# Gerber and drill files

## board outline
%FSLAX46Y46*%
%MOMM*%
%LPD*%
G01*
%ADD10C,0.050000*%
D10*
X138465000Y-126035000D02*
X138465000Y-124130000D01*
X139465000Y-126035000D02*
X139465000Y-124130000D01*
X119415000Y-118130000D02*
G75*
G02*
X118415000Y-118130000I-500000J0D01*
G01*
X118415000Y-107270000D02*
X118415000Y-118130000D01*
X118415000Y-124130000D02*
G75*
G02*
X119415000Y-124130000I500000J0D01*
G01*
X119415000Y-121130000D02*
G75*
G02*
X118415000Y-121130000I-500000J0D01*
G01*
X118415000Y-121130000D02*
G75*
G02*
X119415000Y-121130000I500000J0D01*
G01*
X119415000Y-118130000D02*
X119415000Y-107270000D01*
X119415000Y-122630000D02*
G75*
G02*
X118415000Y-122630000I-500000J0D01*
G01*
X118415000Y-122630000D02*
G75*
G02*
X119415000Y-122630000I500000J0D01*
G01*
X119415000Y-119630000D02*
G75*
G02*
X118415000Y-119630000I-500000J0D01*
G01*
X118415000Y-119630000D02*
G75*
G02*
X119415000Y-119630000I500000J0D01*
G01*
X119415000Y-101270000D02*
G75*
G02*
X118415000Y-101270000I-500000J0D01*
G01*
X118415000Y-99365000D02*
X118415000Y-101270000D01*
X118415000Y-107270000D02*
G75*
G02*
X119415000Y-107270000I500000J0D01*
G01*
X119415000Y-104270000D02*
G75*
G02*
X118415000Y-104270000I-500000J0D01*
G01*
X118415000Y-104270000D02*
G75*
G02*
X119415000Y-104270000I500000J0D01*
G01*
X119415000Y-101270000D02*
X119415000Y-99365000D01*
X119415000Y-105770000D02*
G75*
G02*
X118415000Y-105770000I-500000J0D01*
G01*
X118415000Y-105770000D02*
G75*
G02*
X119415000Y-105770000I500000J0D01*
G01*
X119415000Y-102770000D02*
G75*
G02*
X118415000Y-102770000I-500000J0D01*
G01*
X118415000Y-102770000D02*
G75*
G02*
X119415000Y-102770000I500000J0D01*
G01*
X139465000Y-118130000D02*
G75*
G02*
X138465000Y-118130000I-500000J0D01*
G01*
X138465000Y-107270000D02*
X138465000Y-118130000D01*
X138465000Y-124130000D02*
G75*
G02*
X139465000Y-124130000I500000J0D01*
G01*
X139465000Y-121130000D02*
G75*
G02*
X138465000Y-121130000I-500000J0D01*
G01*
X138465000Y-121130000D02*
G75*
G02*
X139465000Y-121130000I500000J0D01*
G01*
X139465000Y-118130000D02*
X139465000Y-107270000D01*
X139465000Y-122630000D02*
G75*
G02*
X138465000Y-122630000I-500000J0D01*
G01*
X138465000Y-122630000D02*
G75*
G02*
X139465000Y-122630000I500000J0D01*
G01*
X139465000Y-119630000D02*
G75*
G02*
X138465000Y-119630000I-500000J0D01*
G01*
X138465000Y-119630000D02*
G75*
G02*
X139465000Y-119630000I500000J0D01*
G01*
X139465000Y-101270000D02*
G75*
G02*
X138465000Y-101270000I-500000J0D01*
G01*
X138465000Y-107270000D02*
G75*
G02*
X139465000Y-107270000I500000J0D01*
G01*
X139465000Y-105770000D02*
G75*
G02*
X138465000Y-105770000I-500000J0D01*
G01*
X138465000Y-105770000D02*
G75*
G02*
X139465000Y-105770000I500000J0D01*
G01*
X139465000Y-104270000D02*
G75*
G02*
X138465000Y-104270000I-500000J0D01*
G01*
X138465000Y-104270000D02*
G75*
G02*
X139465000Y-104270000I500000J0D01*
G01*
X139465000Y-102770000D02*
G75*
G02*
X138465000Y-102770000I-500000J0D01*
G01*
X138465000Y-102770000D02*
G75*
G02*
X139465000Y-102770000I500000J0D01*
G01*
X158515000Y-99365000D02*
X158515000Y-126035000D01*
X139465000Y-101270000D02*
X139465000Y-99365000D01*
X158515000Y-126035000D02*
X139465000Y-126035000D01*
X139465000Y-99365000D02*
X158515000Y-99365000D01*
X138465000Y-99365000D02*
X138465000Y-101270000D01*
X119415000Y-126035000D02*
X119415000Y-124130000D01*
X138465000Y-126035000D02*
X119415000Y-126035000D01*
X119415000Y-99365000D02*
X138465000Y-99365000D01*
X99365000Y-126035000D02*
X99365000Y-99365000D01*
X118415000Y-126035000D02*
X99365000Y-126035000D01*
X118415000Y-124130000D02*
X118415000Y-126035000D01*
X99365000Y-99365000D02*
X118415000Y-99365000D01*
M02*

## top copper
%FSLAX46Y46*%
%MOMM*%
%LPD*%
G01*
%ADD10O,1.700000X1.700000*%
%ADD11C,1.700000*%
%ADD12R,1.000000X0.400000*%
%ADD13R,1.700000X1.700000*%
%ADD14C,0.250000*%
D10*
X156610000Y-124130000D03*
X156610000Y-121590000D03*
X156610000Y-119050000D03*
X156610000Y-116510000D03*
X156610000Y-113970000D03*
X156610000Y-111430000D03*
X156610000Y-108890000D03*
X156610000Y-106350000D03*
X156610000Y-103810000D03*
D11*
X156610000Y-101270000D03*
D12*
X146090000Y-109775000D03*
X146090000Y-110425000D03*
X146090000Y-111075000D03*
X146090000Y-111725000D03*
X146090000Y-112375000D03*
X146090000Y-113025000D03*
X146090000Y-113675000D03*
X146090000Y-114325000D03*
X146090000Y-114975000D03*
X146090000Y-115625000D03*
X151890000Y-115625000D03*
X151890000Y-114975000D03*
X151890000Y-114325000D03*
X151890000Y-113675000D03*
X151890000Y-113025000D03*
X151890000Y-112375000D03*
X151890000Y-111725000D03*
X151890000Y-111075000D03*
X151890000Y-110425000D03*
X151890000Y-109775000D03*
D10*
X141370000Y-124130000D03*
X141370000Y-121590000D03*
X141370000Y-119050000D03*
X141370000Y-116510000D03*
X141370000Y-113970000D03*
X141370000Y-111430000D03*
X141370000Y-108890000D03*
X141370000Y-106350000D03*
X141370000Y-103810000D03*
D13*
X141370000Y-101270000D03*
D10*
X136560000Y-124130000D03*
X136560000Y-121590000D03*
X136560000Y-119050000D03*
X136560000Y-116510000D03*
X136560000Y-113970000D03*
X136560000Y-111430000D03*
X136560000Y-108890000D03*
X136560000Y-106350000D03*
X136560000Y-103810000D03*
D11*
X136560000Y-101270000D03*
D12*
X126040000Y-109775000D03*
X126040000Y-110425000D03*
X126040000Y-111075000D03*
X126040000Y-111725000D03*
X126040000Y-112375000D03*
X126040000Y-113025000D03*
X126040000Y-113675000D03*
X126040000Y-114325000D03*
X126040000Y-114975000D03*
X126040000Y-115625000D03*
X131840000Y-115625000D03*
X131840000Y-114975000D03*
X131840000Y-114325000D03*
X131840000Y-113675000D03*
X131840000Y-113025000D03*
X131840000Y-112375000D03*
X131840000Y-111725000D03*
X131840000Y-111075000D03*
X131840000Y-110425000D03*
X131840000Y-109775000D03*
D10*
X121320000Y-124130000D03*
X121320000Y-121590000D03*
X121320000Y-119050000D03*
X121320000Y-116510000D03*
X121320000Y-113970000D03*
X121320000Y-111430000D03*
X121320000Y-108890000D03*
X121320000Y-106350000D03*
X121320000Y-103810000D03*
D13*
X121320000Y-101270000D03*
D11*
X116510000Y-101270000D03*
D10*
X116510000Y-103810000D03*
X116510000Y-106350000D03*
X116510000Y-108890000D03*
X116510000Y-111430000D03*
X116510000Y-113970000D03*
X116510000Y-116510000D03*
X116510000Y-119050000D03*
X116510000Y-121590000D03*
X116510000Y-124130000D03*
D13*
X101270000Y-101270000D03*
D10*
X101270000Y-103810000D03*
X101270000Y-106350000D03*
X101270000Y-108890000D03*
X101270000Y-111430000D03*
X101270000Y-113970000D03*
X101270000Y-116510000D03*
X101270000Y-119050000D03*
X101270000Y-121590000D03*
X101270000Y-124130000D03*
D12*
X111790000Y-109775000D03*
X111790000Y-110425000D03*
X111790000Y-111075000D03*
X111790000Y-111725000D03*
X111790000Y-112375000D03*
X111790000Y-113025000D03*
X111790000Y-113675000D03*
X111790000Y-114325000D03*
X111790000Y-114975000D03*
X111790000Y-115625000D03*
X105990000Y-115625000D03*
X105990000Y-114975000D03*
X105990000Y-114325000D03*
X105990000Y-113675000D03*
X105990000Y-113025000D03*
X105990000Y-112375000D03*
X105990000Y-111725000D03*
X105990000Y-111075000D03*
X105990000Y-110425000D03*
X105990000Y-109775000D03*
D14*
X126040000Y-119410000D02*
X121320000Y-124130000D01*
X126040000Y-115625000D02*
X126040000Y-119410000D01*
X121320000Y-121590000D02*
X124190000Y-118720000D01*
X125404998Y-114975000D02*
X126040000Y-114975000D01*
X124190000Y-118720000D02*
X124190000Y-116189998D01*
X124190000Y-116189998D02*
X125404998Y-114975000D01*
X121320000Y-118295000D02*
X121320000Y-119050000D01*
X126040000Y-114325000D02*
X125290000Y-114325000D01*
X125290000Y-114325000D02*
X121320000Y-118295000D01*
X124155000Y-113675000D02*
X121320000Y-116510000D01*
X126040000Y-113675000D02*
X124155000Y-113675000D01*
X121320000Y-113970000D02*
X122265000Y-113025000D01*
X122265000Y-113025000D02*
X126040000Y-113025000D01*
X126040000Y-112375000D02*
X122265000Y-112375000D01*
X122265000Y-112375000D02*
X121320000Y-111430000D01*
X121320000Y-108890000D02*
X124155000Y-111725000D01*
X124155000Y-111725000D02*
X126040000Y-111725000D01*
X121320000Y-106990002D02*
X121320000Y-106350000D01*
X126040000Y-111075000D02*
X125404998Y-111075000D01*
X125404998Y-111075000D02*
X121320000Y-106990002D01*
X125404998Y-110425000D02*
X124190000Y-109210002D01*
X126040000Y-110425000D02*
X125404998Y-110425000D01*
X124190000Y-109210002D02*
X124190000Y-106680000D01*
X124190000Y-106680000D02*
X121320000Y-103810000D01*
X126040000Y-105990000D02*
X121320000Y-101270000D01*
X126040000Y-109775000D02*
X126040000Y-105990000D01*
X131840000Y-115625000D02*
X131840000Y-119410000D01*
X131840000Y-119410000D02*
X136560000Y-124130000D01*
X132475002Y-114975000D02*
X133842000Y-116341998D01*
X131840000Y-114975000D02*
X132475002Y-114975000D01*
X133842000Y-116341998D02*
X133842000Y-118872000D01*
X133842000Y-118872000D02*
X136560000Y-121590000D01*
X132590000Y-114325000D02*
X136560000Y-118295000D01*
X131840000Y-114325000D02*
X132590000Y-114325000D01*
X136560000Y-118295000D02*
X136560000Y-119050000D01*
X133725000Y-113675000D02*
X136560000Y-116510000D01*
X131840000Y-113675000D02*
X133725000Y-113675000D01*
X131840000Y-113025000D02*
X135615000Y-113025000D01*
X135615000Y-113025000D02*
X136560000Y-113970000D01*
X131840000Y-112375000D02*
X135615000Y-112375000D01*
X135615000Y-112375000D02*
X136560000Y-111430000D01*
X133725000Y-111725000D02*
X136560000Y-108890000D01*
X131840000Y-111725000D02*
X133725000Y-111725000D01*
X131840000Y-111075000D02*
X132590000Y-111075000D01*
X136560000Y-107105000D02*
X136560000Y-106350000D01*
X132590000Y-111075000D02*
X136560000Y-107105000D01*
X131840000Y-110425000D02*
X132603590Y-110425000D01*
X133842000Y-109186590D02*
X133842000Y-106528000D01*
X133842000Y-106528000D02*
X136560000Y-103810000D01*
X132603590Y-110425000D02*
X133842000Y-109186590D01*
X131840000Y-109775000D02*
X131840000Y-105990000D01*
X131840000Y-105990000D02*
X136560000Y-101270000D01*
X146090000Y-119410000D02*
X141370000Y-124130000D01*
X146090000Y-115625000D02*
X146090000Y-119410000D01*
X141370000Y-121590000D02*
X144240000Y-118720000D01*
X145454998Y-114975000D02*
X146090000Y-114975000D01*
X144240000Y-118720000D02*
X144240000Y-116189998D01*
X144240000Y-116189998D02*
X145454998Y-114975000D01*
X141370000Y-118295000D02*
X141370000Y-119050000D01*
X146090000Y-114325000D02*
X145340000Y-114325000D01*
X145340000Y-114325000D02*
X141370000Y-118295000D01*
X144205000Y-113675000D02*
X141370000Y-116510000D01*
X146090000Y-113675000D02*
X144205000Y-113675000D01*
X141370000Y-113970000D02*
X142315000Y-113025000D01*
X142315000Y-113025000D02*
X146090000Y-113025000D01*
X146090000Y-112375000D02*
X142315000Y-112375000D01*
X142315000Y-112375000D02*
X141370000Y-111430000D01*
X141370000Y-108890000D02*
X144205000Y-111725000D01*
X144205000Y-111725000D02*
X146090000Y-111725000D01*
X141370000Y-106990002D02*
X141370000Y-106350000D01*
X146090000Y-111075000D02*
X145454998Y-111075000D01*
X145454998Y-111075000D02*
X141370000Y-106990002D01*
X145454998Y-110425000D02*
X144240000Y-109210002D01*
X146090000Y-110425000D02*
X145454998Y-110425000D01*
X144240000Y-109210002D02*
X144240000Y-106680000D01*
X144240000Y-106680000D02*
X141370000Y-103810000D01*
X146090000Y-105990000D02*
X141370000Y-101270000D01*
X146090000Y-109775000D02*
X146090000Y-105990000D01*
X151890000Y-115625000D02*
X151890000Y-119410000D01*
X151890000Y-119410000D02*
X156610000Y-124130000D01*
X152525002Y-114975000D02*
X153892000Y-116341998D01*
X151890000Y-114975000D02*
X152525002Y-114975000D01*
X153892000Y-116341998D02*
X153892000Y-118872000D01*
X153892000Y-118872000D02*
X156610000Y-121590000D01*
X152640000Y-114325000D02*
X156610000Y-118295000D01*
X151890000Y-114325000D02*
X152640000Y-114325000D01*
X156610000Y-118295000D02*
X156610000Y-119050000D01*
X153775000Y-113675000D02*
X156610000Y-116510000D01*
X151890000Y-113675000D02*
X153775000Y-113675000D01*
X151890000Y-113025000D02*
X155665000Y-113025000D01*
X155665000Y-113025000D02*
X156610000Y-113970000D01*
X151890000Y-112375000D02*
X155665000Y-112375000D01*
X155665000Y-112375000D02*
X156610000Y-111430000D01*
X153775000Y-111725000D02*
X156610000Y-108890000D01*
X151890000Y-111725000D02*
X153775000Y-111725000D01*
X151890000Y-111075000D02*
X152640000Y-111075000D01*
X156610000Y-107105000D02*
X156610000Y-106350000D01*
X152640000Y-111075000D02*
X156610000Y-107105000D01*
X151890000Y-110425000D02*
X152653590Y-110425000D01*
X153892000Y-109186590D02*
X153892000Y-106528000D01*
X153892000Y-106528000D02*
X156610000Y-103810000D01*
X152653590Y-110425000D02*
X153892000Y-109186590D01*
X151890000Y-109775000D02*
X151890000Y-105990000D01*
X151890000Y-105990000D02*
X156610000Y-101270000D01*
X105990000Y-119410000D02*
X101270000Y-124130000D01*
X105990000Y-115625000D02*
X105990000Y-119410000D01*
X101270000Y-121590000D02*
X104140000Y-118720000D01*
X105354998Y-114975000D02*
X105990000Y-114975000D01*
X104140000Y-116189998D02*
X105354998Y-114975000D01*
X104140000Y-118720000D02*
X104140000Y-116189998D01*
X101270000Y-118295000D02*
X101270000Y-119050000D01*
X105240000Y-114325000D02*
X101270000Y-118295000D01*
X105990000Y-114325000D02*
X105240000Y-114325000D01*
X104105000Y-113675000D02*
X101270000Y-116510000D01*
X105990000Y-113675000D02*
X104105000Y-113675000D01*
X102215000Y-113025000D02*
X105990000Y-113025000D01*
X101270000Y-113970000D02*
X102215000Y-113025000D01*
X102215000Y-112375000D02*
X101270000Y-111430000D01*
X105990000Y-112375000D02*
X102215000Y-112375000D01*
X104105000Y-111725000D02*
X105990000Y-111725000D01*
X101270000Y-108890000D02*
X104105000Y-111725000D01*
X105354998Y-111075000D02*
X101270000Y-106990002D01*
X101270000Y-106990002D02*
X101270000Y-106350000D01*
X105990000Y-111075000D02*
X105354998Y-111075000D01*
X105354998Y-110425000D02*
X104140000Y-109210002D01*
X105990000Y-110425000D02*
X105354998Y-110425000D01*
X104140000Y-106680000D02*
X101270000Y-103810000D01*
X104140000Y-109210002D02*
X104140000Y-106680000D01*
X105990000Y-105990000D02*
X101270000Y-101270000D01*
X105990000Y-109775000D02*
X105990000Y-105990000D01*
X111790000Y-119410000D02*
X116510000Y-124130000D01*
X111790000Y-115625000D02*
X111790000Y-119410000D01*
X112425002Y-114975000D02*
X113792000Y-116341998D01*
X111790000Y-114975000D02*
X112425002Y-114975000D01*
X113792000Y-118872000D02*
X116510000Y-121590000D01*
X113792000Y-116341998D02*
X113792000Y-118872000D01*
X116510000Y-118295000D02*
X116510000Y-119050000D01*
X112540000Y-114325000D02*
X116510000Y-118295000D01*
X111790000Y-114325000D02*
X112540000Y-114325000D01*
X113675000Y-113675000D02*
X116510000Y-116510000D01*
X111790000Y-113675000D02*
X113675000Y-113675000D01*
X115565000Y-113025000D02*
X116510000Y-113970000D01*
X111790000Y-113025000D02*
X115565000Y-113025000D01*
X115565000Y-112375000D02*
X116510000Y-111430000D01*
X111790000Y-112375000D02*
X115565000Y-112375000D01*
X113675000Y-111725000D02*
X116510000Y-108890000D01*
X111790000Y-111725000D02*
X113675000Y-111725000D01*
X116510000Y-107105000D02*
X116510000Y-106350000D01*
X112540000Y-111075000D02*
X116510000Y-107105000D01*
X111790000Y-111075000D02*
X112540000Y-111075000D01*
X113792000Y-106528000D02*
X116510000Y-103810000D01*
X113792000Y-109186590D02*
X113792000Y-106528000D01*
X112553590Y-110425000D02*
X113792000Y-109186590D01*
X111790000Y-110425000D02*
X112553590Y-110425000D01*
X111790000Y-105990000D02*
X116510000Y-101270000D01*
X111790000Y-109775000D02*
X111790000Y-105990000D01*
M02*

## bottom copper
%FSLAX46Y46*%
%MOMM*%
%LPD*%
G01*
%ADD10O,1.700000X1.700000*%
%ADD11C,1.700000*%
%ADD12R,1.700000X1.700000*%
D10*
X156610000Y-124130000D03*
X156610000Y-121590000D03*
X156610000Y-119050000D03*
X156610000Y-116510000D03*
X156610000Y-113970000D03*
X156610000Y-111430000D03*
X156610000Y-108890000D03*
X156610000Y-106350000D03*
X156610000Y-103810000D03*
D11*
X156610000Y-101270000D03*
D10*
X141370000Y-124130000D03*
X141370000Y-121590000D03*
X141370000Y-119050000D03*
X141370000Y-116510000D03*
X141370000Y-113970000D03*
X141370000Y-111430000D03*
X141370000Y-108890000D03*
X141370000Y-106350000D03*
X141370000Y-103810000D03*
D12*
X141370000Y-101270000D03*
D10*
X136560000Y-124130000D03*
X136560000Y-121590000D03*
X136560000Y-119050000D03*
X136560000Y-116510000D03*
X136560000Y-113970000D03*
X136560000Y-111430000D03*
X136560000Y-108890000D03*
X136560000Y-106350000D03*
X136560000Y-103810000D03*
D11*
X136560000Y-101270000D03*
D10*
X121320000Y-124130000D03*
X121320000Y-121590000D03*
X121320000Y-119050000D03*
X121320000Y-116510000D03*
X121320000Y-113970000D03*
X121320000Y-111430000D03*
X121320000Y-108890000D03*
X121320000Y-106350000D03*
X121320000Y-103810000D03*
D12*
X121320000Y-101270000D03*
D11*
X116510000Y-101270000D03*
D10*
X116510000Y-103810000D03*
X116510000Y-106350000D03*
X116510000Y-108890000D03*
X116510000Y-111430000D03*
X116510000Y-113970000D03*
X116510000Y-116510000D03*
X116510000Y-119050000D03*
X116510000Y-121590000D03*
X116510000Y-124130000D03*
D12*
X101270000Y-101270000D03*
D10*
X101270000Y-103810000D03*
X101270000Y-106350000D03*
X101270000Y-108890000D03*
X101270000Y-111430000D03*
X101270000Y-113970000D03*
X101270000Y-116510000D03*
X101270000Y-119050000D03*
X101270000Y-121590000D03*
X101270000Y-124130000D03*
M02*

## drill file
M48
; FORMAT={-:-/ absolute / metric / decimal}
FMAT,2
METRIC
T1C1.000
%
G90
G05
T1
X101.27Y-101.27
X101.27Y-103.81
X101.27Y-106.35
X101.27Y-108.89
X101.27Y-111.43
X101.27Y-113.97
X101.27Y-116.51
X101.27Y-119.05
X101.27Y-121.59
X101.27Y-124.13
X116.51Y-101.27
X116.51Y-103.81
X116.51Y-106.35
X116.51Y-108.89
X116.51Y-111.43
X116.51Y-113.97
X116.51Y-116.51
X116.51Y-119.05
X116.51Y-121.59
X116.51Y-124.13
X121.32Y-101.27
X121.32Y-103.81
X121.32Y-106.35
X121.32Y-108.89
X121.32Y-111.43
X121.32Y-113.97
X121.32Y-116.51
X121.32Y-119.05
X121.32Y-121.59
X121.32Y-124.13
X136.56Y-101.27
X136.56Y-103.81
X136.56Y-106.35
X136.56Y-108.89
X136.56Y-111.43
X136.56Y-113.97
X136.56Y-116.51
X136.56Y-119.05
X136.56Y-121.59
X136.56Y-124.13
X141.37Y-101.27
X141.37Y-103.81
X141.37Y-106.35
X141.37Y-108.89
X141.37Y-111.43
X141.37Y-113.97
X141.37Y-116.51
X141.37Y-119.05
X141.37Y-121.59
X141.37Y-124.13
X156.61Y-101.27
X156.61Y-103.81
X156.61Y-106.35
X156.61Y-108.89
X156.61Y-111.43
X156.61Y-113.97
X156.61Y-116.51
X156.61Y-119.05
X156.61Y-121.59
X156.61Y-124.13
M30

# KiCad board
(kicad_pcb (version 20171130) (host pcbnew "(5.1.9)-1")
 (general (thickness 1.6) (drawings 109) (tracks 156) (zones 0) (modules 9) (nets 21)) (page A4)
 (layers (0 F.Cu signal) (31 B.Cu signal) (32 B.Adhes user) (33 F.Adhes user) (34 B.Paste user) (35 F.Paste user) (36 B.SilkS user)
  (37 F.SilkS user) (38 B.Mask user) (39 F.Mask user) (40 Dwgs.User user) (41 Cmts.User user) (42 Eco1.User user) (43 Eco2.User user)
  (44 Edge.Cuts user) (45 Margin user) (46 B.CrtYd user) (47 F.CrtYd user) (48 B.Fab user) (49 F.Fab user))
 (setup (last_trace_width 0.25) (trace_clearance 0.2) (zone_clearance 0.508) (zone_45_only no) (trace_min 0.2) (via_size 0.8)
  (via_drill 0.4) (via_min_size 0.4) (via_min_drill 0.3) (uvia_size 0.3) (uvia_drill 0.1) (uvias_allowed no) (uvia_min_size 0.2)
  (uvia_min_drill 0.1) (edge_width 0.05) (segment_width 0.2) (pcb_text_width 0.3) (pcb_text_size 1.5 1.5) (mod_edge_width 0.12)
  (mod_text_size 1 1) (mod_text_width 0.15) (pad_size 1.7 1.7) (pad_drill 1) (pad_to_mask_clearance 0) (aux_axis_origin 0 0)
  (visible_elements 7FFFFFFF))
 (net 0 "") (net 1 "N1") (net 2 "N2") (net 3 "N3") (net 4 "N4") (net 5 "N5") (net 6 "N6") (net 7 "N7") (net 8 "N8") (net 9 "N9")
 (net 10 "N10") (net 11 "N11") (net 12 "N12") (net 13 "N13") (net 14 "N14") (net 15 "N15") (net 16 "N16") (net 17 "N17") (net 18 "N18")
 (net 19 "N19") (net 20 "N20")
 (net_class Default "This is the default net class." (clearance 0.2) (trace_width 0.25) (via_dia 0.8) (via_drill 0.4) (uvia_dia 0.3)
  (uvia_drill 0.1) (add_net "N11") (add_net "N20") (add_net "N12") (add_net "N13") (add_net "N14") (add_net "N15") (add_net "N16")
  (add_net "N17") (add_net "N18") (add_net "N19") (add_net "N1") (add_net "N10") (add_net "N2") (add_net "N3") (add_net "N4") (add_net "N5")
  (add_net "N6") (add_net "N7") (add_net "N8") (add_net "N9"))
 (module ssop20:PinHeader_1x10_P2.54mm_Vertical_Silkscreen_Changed (layer B.Cu) (at 156.61 101.27 180)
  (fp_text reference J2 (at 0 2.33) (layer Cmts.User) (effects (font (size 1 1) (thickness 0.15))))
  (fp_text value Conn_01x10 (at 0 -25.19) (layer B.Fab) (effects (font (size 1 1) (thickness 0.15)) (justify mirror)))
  (pad 10 thru_hole oval (at 0 -22.86 180) (size 1.7 1.7) (drill 1) (layers *.Cu *.Mask))
  (pad 9 thru_hole oval (at 0 -20.32 180) (size 1.7 1.7) (drill 1) (layers *.Cu *.Mask))
  (pad 8 thru_hole oval (at 0 -17.78 180) (size 1.7 1.7) (drill 1) (layers *.Cu *.Mask))
  (pad 7 thru_hole oval (at 0 -15.24 180) (size 1.7 1.7) (drill 1) (layers *.Cu *.Mask))
  (pad 6 thru_hole oval (at 0 -12.7 180) (size 1.7 1.7) (drill 1) (layers *.Cu *.Mask))
  (pad 5 thru_hole oval (at 0 -10.16 180) (size 1.7 1.7) (drill 1) (layers *.Cu *.Mask))
  (pad 4 thru_hole oval (at 0 -7.62 180) (size 1.7 1.7) (drill 1) (layers *.Cu *.Mask))
  (pad 3 thru_hole oval (at 0 -5.08 180) (size 1.7 1.7) (drill 1) (layers *.Cu *.Mask))
  (pad 2 thru_hole oval (at 0 -2.54 180) (size 1.7 1.7) (drill 1) (layers *.Cu *.Mask))
  (pad 1 thru_hole circle (at 0 0 180) (size 1.7 1.7) (drill 1) (layers *.Cu *.Mask)))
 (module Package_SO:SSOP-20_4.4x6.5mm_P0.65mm (layer F.Cu) (at 148.99 112.7)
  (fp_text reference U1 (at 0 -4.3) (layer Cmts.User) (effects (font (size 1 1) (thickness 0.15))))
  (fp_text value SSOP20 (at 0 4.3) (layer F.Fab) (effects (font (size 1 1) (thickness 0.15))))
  (pad 1 smd rect (at -2.9 -2.925) (size 1 0.4) (layers F.Cu F.Paste F.Mask))
  (pad 2 smd rect (at -2.9 -2.275) (size 1 0.4) (layers F.Cu F.Paste F.Mask))
  (pad 3 smd rect (at -2.9 -1.625) (size 1 0.4) (layers F.Cu F.Paste F.Mask))
  (pad 4 smd rect (at -2.9 -0.975) (size 1 0.4) (layers F.Cu F.Paste F.Mask))
  (pad 5 smd rect (at -2.9 -0.325) (size 1 0.4) (layers F.Cu F.Paste F.Mask))
  (pad 6 smd rect (at -2.9 0.325) (size 1 0.4) (layers F.Cu F.Paste F.Mask))
  (pad 7 smd rect (at -2.9 0.975) (size 1 0.4) (layers F.Cu F.Paste F.Mask))
  (pad 8 smd rect (at -2.9 1.625) (size 1 0.4) (layers F.Cu F.Paste F.Mask))
  (pad 9 smd rect (at -2.9 2.275) (size 1 0.4) (layers F.Cu F.Paste F.Mask))
  (pad 10 smd rect (at -2.9 2.925) (size 1 0.4) (layers F.Cu F.Paste F.Mask))
  (pad 11 smd rect (at 2.9 2.925) (size 1 0.4) (layers F.Cu F.Paste F.Mask))
  (pad 12 smd rect (at 2.9 2.275) (size 1 0.4) (layers F.Cu F.Paste F.Mask))
  (pad 13 smd rect (at 2.9 1.625) (size 1 0.4) (layers F.Cu F.Paste F.Mask))
  (pad 14 smd rect (at 2.9 0.975) (size 1 0.4) (layers F.Cu F.Paste F.Mask))
  (pad 15 smd rect (at 2.9 0.325) (size 1 0.4) (layers F.Cu F.Paste F.Mask))
  (pad 16 smd rect (at 2.9 -0.325) (size 1 0.4) (layers F.Cu F.Paste F.Mask))
  (pad 17 smd rect (at 2.9 -0.975) (size 1 0.4) (layers F.Cu F.Paste F.Mask))
  (pad 18 smd rect (at 2.9 -1.625) (size 1 0.4) (layers F.Cu F.Paste F.Mask))
  (pad 19 smd rect (at 2.9 -2.275) (size 1 0.4) (layers F.Cu F.Paste F.Mask))
  (pad 20 smd rect (at 2.9 -2.925) (size 1 0.4) (layers F.Cu F.Paste F.Mask)))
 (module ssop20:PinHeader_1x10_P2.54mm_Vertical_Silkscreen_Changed (layer B.Cu) (at 141.37 101.27 180)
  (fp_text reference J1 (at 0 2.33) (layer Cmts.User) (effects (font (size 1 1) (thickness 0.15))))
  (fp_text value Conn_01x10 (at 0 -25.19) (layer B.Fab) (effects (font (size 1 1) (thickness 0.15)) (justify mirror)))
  (pad 10 thru_hole oval (at 0 -22.86 180) (size 1.7 1.7) (drill 1) (layers *.Cu *.Mask))
  (pad 9 thru_hole oval (at 0 -20.32 180) (size 1.7 1.7) (drill 1) (layers *.Cu *.Mask))
  (pad 8 thru_hole oval (at 0 -17.78 180) (size 1.7 1.7) (drill 1) (layers *.Cu *.Mask))
  (pad 7 thru_hole oval (at 0 -15.24 180) (size 1.7 1.7) (drill 1) (layers *.Cu *.Mask))
  (pad 6 thru_hole oval (at 0 -12.7 180) (size 1.7 1.7) (drill 1) (layers *.Cu *.Mask))
  (pad 5 thru_hole oval (at 0 -10.16 180) (size 1.7 1.7) (drill 1) (layers *.Cu *.Mask))
  (pad 4 thru_hole oval (at 0 -7.62 180) (size 1.7 1.7) (drill 1) (layers *.Cu *.Mask))
  (pad 3 thru_hole oval (at 0 -5.08 180) (size 1.7 1.7) (drill 1) (layers *.Cu *.Mask))
  (pad 2 thru_hole oval (at 0 -2.54 180) (size 1.7 1.7) (drill 1) (layers *.Cu *.Mask))
  (pad 1 thru_hole rect (at 0 0 180) (size 1.7 1.7) (drill 1) (layers *.Cu *.Mask)))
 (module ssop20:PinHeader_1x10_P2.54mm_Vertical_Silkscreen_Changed (layer B.Cu) (at 136.56 101.27 180)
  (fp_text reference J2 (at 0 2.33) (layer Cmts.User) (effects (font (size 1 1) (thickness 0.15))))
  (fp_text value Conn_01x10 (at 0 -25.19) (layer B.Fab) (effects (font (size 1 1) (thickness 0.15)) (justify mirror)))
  (pad 10 thru_hole oval (at 0 -22.86 180) (size 1.7 1.7) (drill 1) (layers *.Cu *.Mask))
  (pad 9 thru_hole oval (at 0 -20.32 180) (size 1.7 1.7) (drill 1) (layers *.Cu *.Mask))
  (pad 8 thru_hole oval (at 0 -17.78 180) (size 1.7 1.7) (drill 1) (layers *.Cu *.Mask))
  (pad 7 thru_hole oval (at 0 -15.24 180) (size 1.7 1.7) (drill 1) (layers *.Cu *.Mask))
  (pad 6 thru_hole oval (at 0 -12.7 180) (size 1.7 1.7) (drill 1) (layers *.Cu *.Mask))
  (pad 5 thru_hole oval (at 0 -10.16 180) (size 1.7 1.7) (drill 1) (layers *.Cu *.Mask))
  (pad 4 thru_hole oval (at 0 -7.62 180) (size 1.7 1.7) (drill 1) (layers *.Cu *.Mask))
  (pad 3 thru_hole oval (at 0 -5.08 180) (size 1.7 1.7) (drill 1) (layers *.Cu *.Mask))
  (pad 2 thru_hole oval (at 0 -2.54 180) (size 1.7 1.7) (drill 1) (layers *.Cu *.Mask))
  (pad 1 thru_hole circle (at 0 0 180) (size 1.7 1.7) (drill 1) (layers *.Cu *.Mask)))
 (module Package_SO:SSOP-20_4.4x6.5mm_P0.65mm (layer F.Cu) (at 128.94 112.7)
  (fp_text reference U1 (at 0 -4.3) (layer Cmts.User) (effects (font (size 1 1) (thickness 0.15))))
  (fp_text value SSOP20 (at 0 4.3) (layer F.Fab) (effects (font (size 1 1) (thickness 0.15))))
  (pad 1 smd rect (at -2.9 -2.925) (size 1 0.4) (layers F.Cu F.Paste F.Mask))
  (pad 2 smd rect (at -2.9 -2.275) (size 1 0.4) (layers F.Cu F.Paste F.Mask))
  (pad 3 smd rect (at -2.9 -1.625) (size 1 0.4) (layers F.Cu F.Paste F.Mask))
  (pad 4 smd rect (at -2.9 -0.975) (size 1 0.4) (layers F.Cu F.Paste F.Mask))
  (pad 5 smd rect (at -2.9 -0.325) (size 1 0.4) (layers F.Cu F.Paste F.Mask))
  (pad 6 smd rect (at -2.9 0.325) (size 1 0.4) (layers F.Cu F.Paste F.Mask))
  (pad 7 smd rect (at -2.9 0.975) (size 1 0.4) (layers F.Cu F.Paste F.Mask))
  (pad 8 smd rect (at -2.9 1.625) (size 1 0.4) (layers F.Cu F.Paste F.Mask))
  (pad 9 smd rect (at -2.9 2.275) (size 1 0.4) (layers F.Cu F.Paste F.Mask))
  (pad 10 smd rect (at -2.9 2.925) (size 1 0.4) (layers F.Cu F.Paste F.Mask))
  (pad 11 smd rect (at 2.9 2.925) (size 1 0.4) (layers F.Cu F.Paste F.Mask))
  (pad 12 smd rect (at 2.9 2.275) (size 1 0.4) (layers F.Cu F.Paste F.Mask))
  (pad 13 smd rect (at 2.9 1.625) (size 1 0.4) (layers F.Cu F.Paste F.Mask))
  (pad 14 smd rect (at 2.9 0.975) (size 1 0.4) (layers F.Cu F.Paste F.Mask))
  (pad 15 smd rect (at 2.9 0.325) (size 1 0.4) (layers F.Cu F.Paste F.Mask))
  (pad 16 smd rect (at 2.9 -0.325) (size 1 0.4) (layers F.Cu F.Paste F.Mask))
  (pad 17 smd rect (at 2.9 -0.975) (size 1 0.4) (layers F.Cu F.Paste F.Mask))
  (pad 18 smd rect (at 2.9 -1.625) (size 1 0.4) (layers F.Cu F.Paste F.Mask))
  (pad 19 smd rect (at 2.9 -2.275) (size 1 0.4) (layers F.Cu F.Paste F.Mask))
  (pad 20 smd rect (at 2.9 -2.925) (size 1 0.4) (layers F.Cu F.Paste F.Mask)))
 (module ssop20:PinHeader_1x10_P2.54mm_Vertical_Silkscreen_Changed (layer B.Cu) (at 121.32 101.27 180)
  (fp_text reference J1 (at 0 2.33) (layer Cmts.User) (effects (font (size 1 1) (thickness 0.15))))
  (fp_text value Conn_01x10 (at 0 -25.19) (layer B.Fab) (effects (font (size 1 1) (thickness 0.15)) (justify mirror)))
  (pad 10 thru_hole oval (at 0 -22.86 180) (size 1.7 1.7) (drill 1) (layers *.Cu *.Mask))
  (pad 9 thru_hole oval (at 0 -20.32 180) (size 1.7 1.7) (drill 1) (layers *.Cu *.Mask))
  (pad 8 thru_hole oval (at 0 -17.78 180) (size 1.7 1.7) (drill 1) (layers *.Cu *.Mask))
  (pad 7 thru_hole oval (at 0 -15.24 180) (size 1.7 1.7) (drill 1) (layers *.Cu *.Mask))
  (pad 6 thru_hole oval (at 0 -12.7 180) (size 1.7 1.7) (drill 1) (layers *.Cu *.Mask))
  (pad 5 thru_hole oval (at 0 -10.16 180) (size 1.7 1.7) (drill 1) (layers *.Cu *.Mask))
  (pad 4 thru_hole oval (at 0 -7.62 180) (size 1.7 1.7) (drill 1) (layers *.Cu *.Mask))
  (pad 3 thru_hole oval (at 0 -5.08 180) (size 1.7 1.7) (drill 1) (layers *.Cu *.Mask))
  (pad 2 thru_hole oval (at 0 -2.54 180) (size 1.7 1.7) (drill 1) (layers *.Cu *.Mask))
  (pad 1 thru_hole rect (at 0 0 180) (size 1.7 1.7) (drill 1) (layers *.Cu *.Mask)))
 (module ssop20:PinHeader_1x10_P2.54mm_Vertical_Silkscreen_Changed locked (layer B.Cu) (at 116.51 101.27 180)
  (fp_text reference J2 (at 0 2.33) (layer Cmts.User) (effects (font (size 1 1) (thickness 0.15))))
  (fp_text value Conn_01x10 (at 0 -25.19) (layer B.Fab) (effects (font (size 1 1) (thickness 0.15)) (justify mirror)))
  (pad 1 thru_hole circle (at 0 0 180) (size 1.7 1.7) (drill 1) (layers *.Cu *.Mask) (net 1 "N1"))
  (pad 2 thru_hole oval (at 0 -2.54 180) (size 1.7 1.7) (drill 1) (layers *.Cu *.Mask) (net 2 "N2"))
  (pad 3 thru_hole oval (at 0 -5.08 180) (size 1.7 1.7) (drill 1) (layers *.Cu *.Mask) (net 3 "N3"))
  (pad 4 thru_hole oval (at 0 -7.62 180) (size 1.7 1.7) (drill 1) (layers *.Cu *.Mask) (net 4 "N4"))
  (pad 5 thru_hole oval (at 0 -10.16 180) (size 1.7 1.7) (drill 1) (layers *.Cu *.Mask) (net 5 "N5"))
  (pad 6 thru_hole oval (at 0 -12.7 180) (size 1.7 1.7) (drill 1) (layers *.Cu *.Mask) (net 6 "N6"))
  (pad 7 thru_hole oval (at 0 -15.24 180) (size 1.7 1.7) (drill 1) (layers *.Cu *.Mask) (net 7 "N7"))
  (pad 8 thru_hole oval (at 0 -17.78 180) (size 1.7 1.7) (drill 1) (layers *.Cu *.Mask) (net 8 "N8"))
  (pad 9 thru_hole oval (at 0 -20.32 180) (size 1.7 1.7) (drill 1) (layers *.Cu *.Mask) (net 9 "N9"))
  (pad 10 thru_hole oval (at 0 -22.86 180) (size 1.7 1.7) (drill 1) (layers *.Cu *.Mask) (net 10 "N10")))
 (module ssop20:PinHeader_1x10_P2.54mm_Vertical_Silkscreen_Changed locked (layer B.Cu) (at 101.27 101.27 180)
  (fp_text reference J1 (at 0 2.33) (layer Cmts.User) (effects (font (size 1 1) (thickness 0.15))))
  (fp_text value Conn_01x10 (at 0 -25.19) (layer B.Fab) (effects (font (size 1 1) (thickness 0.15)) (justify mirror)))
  (pad 1 thru_hole rect (at 0 0 180) (size 1.7 1.7) (drill 1) (layers *.Cu *.Mask) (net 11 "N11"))
  (pad 2 thru_hole oval (at 0 -2.54 180) (size 1.7 1.7) (drill 1) (layers *.Cu *.Mask) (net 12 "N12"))
  (pad 3 thru_hole oval (at 0 -5.08 180) (size 1.7 1.7) (drill 1) (layers *.Cu *.Mask) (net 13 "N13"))
  (pad 4 thru_hole oval (at 0 -7.62 180) (size 1.7 1.7) (drill 1) (layers *.Cu *.Mask) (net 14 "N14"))
  (pad 5 thru_hole oval (at 0 -10.16 180) (size 1.7 1.7) (drill 1) (layers *.Cu *.Mask) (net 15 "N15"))
  (pad 6 thru_hole oval (at 0 -12.7 180) (size 1.7 1.7) (drill 1) (layers *.Cu *.Mask) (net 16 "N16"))
  (pad 7 thru_hole oval (at 0 -15.24 180) (size 1.7 1.7) (drill 1) (layers *.Cu *.Mask) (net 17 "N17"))
  (pad 8 thru_hole oval (at 0 -17.78 180) (size 1.7 1.7) (drill 1) (layers *.Cu *.Mask) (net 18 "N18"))
  (pad 9 thru_hole oval (at 0 -20.32 180) (size 1.7 1.7) (drill 1) (layers *.Cu *.Mask) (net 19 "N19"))
  (pad 10 thru_hole oval (at 0 -22.86 180) (size 1.7 1.7) (drill 1) (layers *.Cu *.Mask) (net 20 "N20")))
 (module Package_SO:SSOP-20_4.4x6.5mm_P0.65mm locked (layer F.Cu) (at 108.89 112.7)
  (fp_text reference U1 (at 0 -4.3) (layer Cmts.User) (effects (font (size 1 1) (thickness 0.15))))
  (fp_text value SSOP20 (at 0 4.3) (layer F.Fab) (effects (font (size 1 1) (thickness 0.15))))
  (pad 20 smd rect (at 2.9 -2.925) (size 1 0.4) (layers F.Cu F.Paste F.Mask) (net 1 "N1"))
  (pad 19 smd rect (at 2.9 -2.275) (size 1 0.4) (layers F.Cu F.Paste F.Mask) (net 2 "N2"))
  (pad 18 smd rect (at 2.9 -1.625) (size 1 0.4) (layers F.Cu F.Paste F.Mask) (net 3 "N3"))
  (pad 17 smd rect (at 2.9 -0.975) (size 1 0.4) (layers F.Cu F.Paste F.Mask) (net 4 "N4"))
  (pad 16 smd rect (at 2.9 -0.325) (size 1 0.4) (layers F.Cu F.Paste F.Mask) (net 5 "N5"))
  (pad 15 smd rect (at 2.9 0.325) (size 1 0.4) (layers F.Cu F.Paste F.Mask) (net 6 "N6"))
  (pad 14 smd rect (at 2.9 0.975) (size 1 0.4) (layers F.Cu F.Paste F.Mask) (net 7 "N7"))
  (pad 13 smd rect (at 2.9 1.625) (size 1 0.4) (layers F.Cu F.Paste F.Mask) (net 8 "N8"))
  (pad 12 smd rect (at 2.9 2.275) (size 1 0.4) (layers F.Cu F.Paste F.Mask) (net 9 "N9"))
  (pad 11 smd rect (at 2.9 2.925) (size 1 0.4) (layers F.Cu F.Paste F.Mask) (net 10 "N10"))
  (pad 10 smd rect (at -2.9 2.925) (size 1 0.4) (layers F.Cu F.Paste F.Mask) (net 20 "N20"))
  (pad 9 smd rect (at -2.9 2.275) (size 1 0.4) (layers F.Cu F.Paste F.Mask) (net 19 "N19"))
  (pad 8 smd rect (at -2.9 1.625) (size 1 0.4) (layers F.Cu F.Paste F.Mask) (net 18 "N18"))
  (pad 7 smd rect (at -2.9 0.975) (size 1 0.4) (layers F.Cu F.Paste F.Mask) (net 17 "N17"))
  (pad 6 smd rect (at -2.9 0.325) (size 1 0.4) (layers F.Cu F.Paste F.Mask) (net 16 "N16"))
  (pad 5 smd rect (at -2.9 -0.325) (size 1 0.4) (layers F.Cu F.Paste F.Mask) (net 15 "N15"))
  (pad 4 smd rect (at -2.9 -0.975) (size 1 0.4) (layers F.Cu F.Paste F.Mask) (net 14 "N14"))
  (pad 3 smd rect (at -2.9 -1.625) (size 1 0.4) (layers F.Cu F.Paste F.Mask) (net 13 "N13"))
  (pad 2 smd rect (at -2.9 -2.275) (size 1 0.4) (layers F.Cu F.Paste F.Mask) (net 12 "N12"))
  (pad 1 smd rect (at -2.9 -2.925) (size 1 0.4) (layers F.Cu F.Paste F.Mask) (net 11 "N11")))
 (gr_line (start 138.465 126.035) (end 138.465 124.13) (layer Edge.Cuts) (width 0.05))
 (gr_line (start 139.465 126.035) (end 139.465 124.13) (layer Edge.Cuts) (width 0.05))
 (gr_arc (start 118.915 118.13) (end 118.415 118.13) (angle -180) (layer Edge.Cuts) (width 0.05))
 (gr_line (start 118.415 107.27) (end 118.415 118.13) (layer Edge.Cuts) (width 0.05))
 (gr_arc (start 118.915 124.13) (end 119.415 124.13) (angle -180) (layer Edge.Cuts) (width 0.05))
 (gr_circle (center 118.915 121.13) (end 119.415 121.13) (layer Edge.Cuts) (width 0.05))
 (gr_line (start 119.415 118.13) (end 119.415 107.27) (layer Edge.Cuts) (width 0.05))
 (gr_circle (center 118.915 122.63) (end 119.415 122.63) (layer Edge.Cuts) (width 0.05))
 (gr_circle (center 118.915 119.63) (end 119.415 119.63) (layer Edge.Cuts) (width 0.05))
 (gr_arc (start 118.915 101.27) (end 118.415 101.27) (angle -180) (layer Edge.Cuts) (width 0.05))
 (gr_line (start 118.415 99.365) (end 118.415 101.27) (layer Edge.Cuts) (width 0.05))
 (gr_arc (start 118.915 107.27) (end 119.415 107.27) (angle -180) (layer Edge.Cuts) (width 0.05))
 (gr_circle (center 118.915 104.27) (end 119.415 104.27) (layer Edge.Cuts) (width 0.05))
 (gr_line (start 119.415 101.27) (end 119.415 99.365) (layer Edge.Cuts) (width 0.05))
 (gr_circle (center 118.915 105.77) (end 119.415 105.77) (layer Edge.Cuts) (width 0.05))
 (gr_circle (center 118.915 102.77) (end 119.415 102.77) (layer Edge.Cuts) (width 0.05))
 (gr_arc (start 138.965 118.13) (end 138.465 118.13) (angle -180) (layer Edge.Cuts) (width 0.05))
 (gr_line (start 138.465 107.27) (end 138.465 118.13) (layer Edge.Cuts) (width 0.05))
 (gr_arc (start 138.965 124.13) (end 139.465 124.13) (angle -180) (layer Edge.Cuts) (width 0.05))
 (gr_circle (center 138.965 121.13) (end 139.465 121.13) (layer Edge.Cuts) (width 0.05))
 (gr_line (start 139.465 118.13) (end 139.465 107.27) (layer Edge.Cuts) (width 0.05))
 (gr_circle (center 138.965 122.63) (end 139.465 122.63) (layer Edge.Cuts) (width 0.05))
 (gr_circle (center 138.965 119.63) (end 139.465 119.63) (layer Edge.Cuts) (width 0.05))
 (gr_arc (start 138.965 101.27) (end 138.465 101.27) (angle -180) (layer Edge.Cuts) (width 0.05))
 (gr_arc (start 138.965 107.27) (end 139.465 107.27) (angle -180) (layer Edge.Cuts) (width 0.05))
 (gr_circle (center 138.965 105.77) (end 139.465 105.77) (layer Edge.Cuts) (width 0.05))
 (gr_circle (center 138.965 104.27) (end 139.465 104.27) (layer Edge.Cuts) (width 0.05))
 (gr_circle (center 138.965 102.77) (end 139.465 102.77) (layer Edge.Cuts) (width 0.05))
 (gr_line (start 158.515 99.365) (end 158.515 126.035) (layer Edge.Cuts) (width 0.05))
 (gr_line (start 139.465 101.27) (end 139.465 99.365) (layer Edge.Cuts) (width 0.05))
 (gr_line (start 158.515 126.035) (end 139.465 126.035) (layer Edge.Cuts) (width 0.05))
 (gr_line (start 139.465 99.365) (end 158.515 99.365) (layer Edge.Cuts) (width 0.05))
 (gr_line (start 138.465 99.365) (end 138.465 101.27) (layer Edge.Cuts) (width 0.05))
 (gr_line (start 119.415 126.035) (end 119.415 124.13) (layer Edge.Cuts) (width 0.05))
 (gr_line (start 138.465 126.035) (end 119.415 126.035) (layer Edge.Cuts) (width 0.05))
 (gr_line (start 119.415 99.365) (end 138.465 99.365) (layer Edge.Cuts) (width 0.05))
 (gr_line (start 99.365 126.035) (end 99.365 99.365) (layer Edge.Cuts) (width 0.05))
 (gr_line (start 118.415 126.035) (end 99.365 126.035) (layer Edge.Cuts) (width 0.05))
 (gr_line (start 118.415 124.13) (end 118.415 126.035) (layer Edge.Cuts) (width 0.05))
 (gr_line (start 99.365 99.365) (end 118.415 99.365) (layer Edge.Cuts) (width 0.05))
 (segment (start 126.04 119.41) (end 121.32 124.13) (width 0.25) (layer F.Cu) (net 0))
 (segment (start 126.04 115.625) (end 126.04 119.41) (width 0.25) (layer F.Cu) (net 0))
 (segment (start 121.32 121.59) (end 124.19 118.72) (width 0.25) (layer F.Cu) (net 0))
 (segment (start 125.404998 114.975) (end 126.04 114.975) (width 0.25) (layer F.Cu) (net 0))
 (segment (start 124.19 118.72) (end 124.19 116.189998) (width 0.25) (layer F.Cu) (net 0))
 (segment (start 124.19 116.189998) (end 125.404998 114.975) (width 0.25) (layer F.Cu) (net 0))
 (segment (start 121.32 118.295) (end 121.32 119.05) (width 0.25) (layer F.Cu) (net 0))
 (segment (start 126.04 114.325) (end 125.29 114.325) (width 0.25) (layer F.Cu) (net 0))
 (segment (start 125.29 114.325) (end 121.32 118.295) (width 0.25) (layer F.Cu) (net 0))
 (segment (start 124.155 113.675) (end 121.32 116.51) (width 0.25) (layer F.Cu) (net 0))
 (segment (start 126.04 113.675) (end 124.155 113.675) (width 0.25) (layer F.Cu) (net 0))
 (segment (start 121.32 113.97) (end 122.265 113.025) (width 0.25) (layer F.Cu) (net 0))
 (segment (start 122.265 113.025) (end 126.04 113.025) (width 0.25) (layer F.Cu) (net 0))
 (segment (start 126.04 112.375) (end 122.265 112.375) (width 0.25) (layer F.Cu) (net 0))
 (segment (start 122.265 112.375) (end 121.32 111.43) (width 0.25) (layer F.Cu) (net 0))
 (segment (start 121.32 108.89) (end 124.155 111.725) (width 0.25) (layer F.Cu) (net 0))
 (segment (start 124.155 111.725) (end 126.04 111.725) (width 0.25) (layer F.Cu) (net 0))
 (segment (start 121.32 106.990002) (end 121.32 106.35) (width 0.25) (layer F.Cu) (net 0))
 (segment (start 126.04 111.075) (end 125.404998 111.075) (width 0.25) (layer F.Cu) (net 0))
 (segment (start 125.404998 111.075) (end 121.32 106.990002) (width 0.25) (layer F.Cu) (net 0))
 (segment (start 125.404998 110.425) (end 124.19 109.210002) (width 0.25) (layer F.Cu) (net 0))
 (segment (start 126.04 110.425) (end 125.404998 110.425) (width 0.25) (layer F.Cu) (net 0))
 (segment (start 124.19 109.210002) (end 124.19 106.68) (width 0.25) (layer F.Cu) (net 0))
 (segment (start 124.19 106.68) (end 121.32 103.81) (width 0.25) (layer F.Cu) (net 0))
 (segment (start 126.04 105.99) (end 121.32 101.27) (width 0.25) (layer F.Cu) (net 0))
 (segment (start 126.04 109.775) (end 126.04 105.99) (width 0.25) (layer F.Cu) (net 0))
 (segment (start 131.84 115.625) (end 131.84 119.41) (width 0.25) (layer F.Cu) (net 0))
 (segment (start 131.84 119.41) (end 136.56 124.13) (width 0.25) (layer F.Cu) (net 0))
 (segment (start 132.475002 114.975) (end 133.842 116.341998) (width 0.25) (layer F.Cu) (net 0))
 (segment (start 131.84 114.975) (end 132.475002 114.975) (width 0.25) (layer F.Cu) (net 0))
 (segment (start 133.842 116.341998) (end 133.842 118.872) (width 0.25) (layer F.Cu) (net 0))
 (segment (start 133.842 118.872) (end 136.56 121.59) (width 0.25) (layer F.Cu) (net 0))
 (segment (start 132.59 114.325) (end 136.56 118.295) (width 0.25) (layer F.Cu) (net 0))
 (segment (start 131.84 114.325) (end 132.59 114.325) (width 0.25) (layer F.Cu) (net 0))
 (segment (start 136.56 118.295) (end 136.56 119.05) (width 0.25) (layer F.Cu) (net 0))
 (segment (start 133.725 113.675) (end 136.56 116.51) (width 0.25) (layer F.Cu) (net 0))
 (segment (start 131.84 113.675) (end 133.725 113.675) (width 0.25) (layer F.Cu) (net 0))
 (segment (start 131.84 113.025) (end 135.615 113.025) (width 0.25) (layer F.Cu) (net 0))
 (segment (start 135.615 113.025) (end 136.56 113.97) (width 0.25) (layer F.Cu) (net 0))
 (segment (start 131.84 112.375) (end 135.615 112.375) (width 0.25) (layer F.Cu) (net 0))
 (segment (start 135.615 112.375) (end 136.56 111.43) (width 0.25) (layer F.Cu) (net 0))
 (segment (start 133.725 111.725) (end 136.56 108.89) (width 0.25) (layer F.Cu) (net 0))
 (segment (start 131.84 111.725) (end 133.725 111.725) (width 0.25) (layer F.Cu) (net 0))
 (segment (start 131.84 111.075) (end 132.59 111.075) (width 0.25) (layer F.Cu) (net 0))
 (segment (start 136.56 107.105) (end 136.56 106.35) (width 0.25) (layer F.Cu) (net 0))
 (segment (start 132.59 111.075) (end 136.56 107.105) (width 0.25) (layer F.Cu) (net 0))
 (segment (start 131.84 110.425) (end 132.60359 110.425) (width 0.25) (layer F.Cu) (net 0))
 (segment (start 133.842 109.18659) (end 133.842 106.528) (width 0.25) (layer F.Cu) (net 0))
 (segment (start 133.842 106.528) (end 136.56 103.81) (width 0.25) (layer F.Cu) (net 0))
 (segment (start 132.60359 110.425) (end 133.842 109.18659) (width 0.25) (layer F.Cu) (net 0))
 (segment (start 131.84 109.775) (end 131.84 105.99) (width 0.25) (layer F.Cu) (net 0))
 (segment (start 131.84 105.99) (end 136.56 101.27) (width 0.25) (layer F.Cu) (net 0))
 (segment (start 146.09 119.41) (end 141.37 124.13) (width 0.25) (layer F.Cu) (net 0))
 (segment (start 146.09 115.625) (end 146.09 119.41) (width 0.25) (layer F.Cu) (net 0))
 (segment (start 141.37 121.59) (end 144.24 118.72) (width 0.25) (layer F.Cu) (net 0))
 (segment (start 145.454998 114.975) (end 146.09 114.975) (width 0.25) (layer F.Cu) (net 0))
 (segment (start 144.24 118.72) (end 144.24 116.189998) (width 0.25) (layer F.Cu) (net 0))
 (segment (start 144.24 116.189998) (end 145.454998 114.975) (width 0.25) (layer F.Cu) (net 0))
 (segment (start 141.37 118.295) (end 141.37 119.05) (width 0.25) (layer F.Cu) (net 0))
 (segment (start 146.09 114.325) (end 145.34 114.325) (width 0.25) (layer F.Cu) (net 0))
 (segment (start 145.34 114.325) (end 141.37 118.295) (width 0.25) (layer F.Cu) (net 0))
 (segment (start 144.205 113.675) (end 141.37 116.51) (width 0.25) (layer F.Cu) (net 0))
 (segment (start 146.09 113.675) (end 144.205 113.675) (width 0.25) (layer F.Cu) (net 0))
 (segment (start 141.37 113.97) (end 142.315 113.025) (width 0.25) (layer F.Cu) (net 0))
 (segment (start 142.315 113.025) (end 146.09 113.025) (width 0.25) (layer F.Cu) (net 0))
 (segment (start 146.09 112.375) (end 142.315 112.375) (width 0.25) (layer F.Cu) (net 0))
 (segment (start 142.315 112.375) (end 141.37 111.43) (width 0.25) (layer F.Cu) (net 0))
 (segment (start 141.37 108.89) (end 144.205 111.725) (width 0.25) (layer F.Cu) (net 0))
 (segment (start 144.205 111.725) (end 146.09 111.725) (width 0.25) (layer F.Cu) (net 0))
 (segment (start 141.37 106.990002) (end 141.37 106.35) (width 0.25) (layer F.Cu) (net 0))
 (segment (start 146.09 111.075) (end 145.454998 111.075) (width 0.25) (layer F.Cu) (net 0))
 (segment (start 145.454998 111.075) (end 141.37 106.990002) (width 0.25) (layer F.Cu) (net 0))
 (segment (start 145.454998 110.425) (end 144.24 109.210002) (width 0.25) (layer F.Cu) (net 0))
 (segment (start 146.09 110.425) (end 145.454998 110.425) (width 0.25) (layer F.Cu) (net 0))
 (segment (start 144.24 109.210002) (end 144.24 106.68) (width 0.25) (layer F.Cu) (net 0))
 (segment (start 144.24 106.68) (end 141.37 103.81) (width 0.25) (layer F.Cu) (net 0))
 (segment (start 146.09 105.99) (end 141.37 101.27) (width 0.25) (layer F.Cu) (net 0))
 (segment (start 146.09 109.775) (end 146.09 105.99) (width 0.25) (layer F.Cu) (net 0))
 (segment (start 151.89 115.625) (end 151.89 119.41) (width 0.25) (layer F.Cu) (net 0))
 (segment (start 151.89 119.41) (end 156.61 124.13) (width 0.25) (layer F.Cu) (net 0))
 (segment (start 152.525002 114.975) (end 153.892 116.341998) (width 0.25) (layer F.Cu) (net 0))
 (segment (start 151.89 114.975) (end 152.525002 114.975) (width 0.25) (layer F.Cu) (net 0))
 (segment (start 153.892 116.341998) (end 153.892 118.872) (width 0.25) (layer F.Cu) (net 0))
 (segment (start 153.892 118.872) (end 156.61 121.59) (width 0.25) (layer F.Cu) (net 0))
 (segment (start 152.64 114.325) (end 156.61 118.295) (width 0.25) (layer F.Cu) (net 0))
 (segment (start 151.89 114.325) (end 152.64 114.325) (width 0.25) (layer F.Cu) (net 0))
 (segment (start 156.61 118.295) (end 156.61 119.05) (width 0.25) (layer F.Cu) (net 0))
 (segment (start 153.775 113.675) (end 156.61 116.51) (width 0.25) (layer F.Cu) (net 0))
 (segment (start 151.89 113.675) (end 153.775 113.675) (width 0.25) (layer F.Cu) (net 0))
 (segment (start 151.89 113.025) (end 155.665 113.025) (width 0.25) (layer F.Cu) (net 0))
 (segment (start 155.665 113.025) (end 156.61 113.97) (width 0.25) (layer F.Cu) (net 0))
 (segment (start 151.89 112.375) (end 155.665 112.375) (width 0.25) (layer F.Cu) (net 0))
 (segment (start 155.665 112.375) (end 156.61 111.43) (width 0.25) (layer F.Cu) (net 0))
 (segment (start 153.775 111.725) (end 156.61 108.89) (width 0.25) (layer F.Cu) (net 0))
 (segment (start 151.89 111.725) (end 153.775 111.725) (width 0.25) (layer F.Cu) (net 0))
 (segment (start 151.89 111.075) (end 152.64 111.075) (width 0.25) (layer F.Cu) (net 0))
 (segment (start 156.61 107.105) (end 156.61 106.35) (width 0.25) (layer F.Cu) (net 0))
 (segment (start 152.64 111.075) (end 156.61 107.105) (width 0.25) (layer F.Cu) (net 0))
 (segment (start 151.89 110.425) (end 152.65359 110.425) (width 0.25) (layer F.Cu) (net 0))
 (segment (start 153.892 109.18659) (end 153.892 106.528) (width 0.25) (layer F.Cu) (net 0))
 (segment (start 153.892 106.528) (end 156.61 103.81) (width 0.25) (layer F.Cu) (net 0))
 (segment (start 152.65359 110.425) (end 153.892 109.18659) (width 0.25) (layer F.Cu) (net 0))
 (segment (start 151.89 109.775) (end 151.89 105.99) (width 0.25) (layer F.Cu) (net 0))
 (segment (start 151.89 105.99) (end 156.61 101.27) (width 0.25) (layer F.Cu) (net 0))
 (segment (start 105.99 119.41) (end 101.27 124.13) (width 0.25) (layer F.Cu) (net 20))
 (segment (start 105.99 115.625) (end 105.99 119.41) (width 0.25) (layer F.Cu) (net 20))
 (segment (start 101.27 121.59) (end 104.14 118.72) (width 0.25) (layer F.Cu) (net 19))
 (segment (start 105.354998 114.975) (end 105.99 114.975) (width 0.25) (layer F.Cu) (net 19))
 (segment (start 104.14 116.189998) (end 105.354998 114.975) (width 0.25) (layer F.Cu) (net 19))
 (segment (start 104.14 118.72) (end 104.14 116.189998) (width 0.25) (layer F.Cu) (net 19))
 (segment (start 101.27 118.295) (end 101.27 119.05) (width 0.25) (layer F.Cu) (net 18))
 (segment (start 105.24 114.325) (end 101.27 118.295) (width 0.25) (layer F.Cu) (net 18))
 (segment (start 105.99 114.325) (end 105.24 114.325) (width 0.25) (layer F.Cu) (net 18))
 (segment (start 104.105 113.675) (end 101.27 116.51) (width 0.25) (layer F.Cu) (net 17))
 (segment (start 105.99 113.675) (end 104.105 113.675) (width 0.25) (layer F.Cu) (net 17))
 (segment (start 102.215 113.025) (end 105.99 113.025) (width 0.25) (layer F.Cu) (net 16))
 (segment (start 101.27 113.97) (end 102.215 113.025) (width 0.25) (layer F.Cu) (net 16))
 (segment (start 102.215 112.375) (end 101.27 111.43) (width 0.25) (layer F.Cu) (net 15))
 (segment (start 105.99 112.375) (end 102.215 112.375) (width 0.25) (layer F.Cu) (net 15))
 (segment (start 104.105 111.725) (end 105.99 111.725) (width 0.25) (layer F.Cu) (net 14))
 (segment (start 101.27 108.89) (end 104.105 111.725) (width 0.25) (layer F.Cu) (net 14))
 (segment (start 105.354998 111.075) (end 101.27 106.990002) (width 0.25) (layer F.Cu) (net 13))
 (segment (start 101.27 106.990002) (end 101.27 106.35) (width 0.25) (layer F.Cu) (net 13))
 (segment (start 105.99 111.075) (end 105.354998 111.075) (width 0.25) (layer F.Cu) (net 13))
 (segment (start 105.354998 110.425) (end 104.14 109.210002) (width 0.25) (layer F.Cu) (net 12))
 (segment (start 105.99 110.425) (end 105.354998 110.425) (width 0.25) (layer F.Cu) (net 12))
 (segment (start 104.14 106.68) (end 101.27 103.81) (width 0.25) (layer F.Cu) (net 12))
 (segment (start 104.14 109.210002) (end 104.14 106.68) (width 0.25) (layer F.Cu) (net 12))
 (segment (start 105.99 105.99) (end 101.27 101.27) (width 0.25) (layer F.Cu) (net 11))
 (segment (start 105.99 109.775) (end 105.99 105.99) (width 0.25) (layer F.Cu) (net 11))
 (segment (start 111.79 119.41) (end 116.51 124.13) (width 0.25) (layer F.Cu) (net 10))
 (segment (start 111.79 115.625) (end 111.79 119.41) (width 0.25) (layer F.Cu) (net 10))
 (segment (start 112.425002 114.975) (end 113.792 116.341998) (width 0.25) (layer F.Cu) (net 9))
 (segment (start 111.79 114.975) (end 112.425002 114.975) (width 0.25) (layer F.Cu) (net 9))
 (segment (start 113.792 118.872) (end 116.51 121.59) (width 0.25) (layer F.Cu) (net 9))
 (segment (start 113.792 116.341998) (end 113.792 118.872) (width 0.25) (layer F.Cu) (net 9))
 (segment (start 116.51 118.295) (end 116.51 119.05) (width 0.25) (layer F.Cu) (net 8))
 (segment (start 112.54 114.325) (end 116.51 118.295) (width 0.25) (layer F.Cu) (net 8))
 (segment (start 111.79 114.325) (end 112.54 114.325) (width 0.25) (layer F.Cu) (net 8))
 (segment (start 113.675 113.675) (end 116.51 116.51) (width 0.25) (layer F.Cu) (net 7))
 (segment (start 111.79 113.675) (end 113.675 113.675) (width 0.25) (layer F.Cu) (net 7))
 (segment (start 115.565 113.025) (end 116.51 113.97) (width 0.25) (layer F.Cu) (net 6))
 (segment (start 111.79 113.025) (end 115.565 113.025) (width 0.25) (layer F.Cu) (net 6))
 (segment (start 115.565 112.375) (end 116.51 111.43) (width 0.25) (layer F.Cu) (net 5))
 (segment (start 111.79 112.375) (end 115.565 112.375) (width 0.25) (layer F.Cu) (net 5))
 (segment (start 113.675 111.725) (end 116.51 108.89) (width 0.25) (layer F.Cu) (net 4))
 (segment (start 111.79 111.725) (end 113.675 111.725) (width 0.25) (layer F.Cu) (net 4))
 (segment (start 116.51 107.105) (end 116.51 106.35) (width 0.25) (layer F.Cu) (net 3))
 (segment (start 112.54 111.075) (end 116.51 107.105) (width 0.25) (layer F.Cu) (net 3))
 (segment (start 111.79 111.075) (end 112.54 111.075) (width 0.25) (layer F.Cu) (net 3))
 (segment (start 113.792 106.528) (end 116.51 103.81) (width 0.25) (layer F.Cu) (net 2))
 (segment (start 113.792 109.18659) (end 113.792 106.528) (width 0.25) (layer F.Cu) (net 2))
 (segment (start 112.55359 110.425) (end 113.792 109.18659) (width 0.25) (layer F.Cu) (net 2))
 (segment (start 111.79 110.425) (end 112.55359 110.425) (width 0.25) (layer F.Cu) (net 2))
 (segment (start 111.79 105.99) (end 116.51 101.27) (width 0.25) (layer F.Cu) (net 1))
 (segment (start 111.79 109.775) (end 111.79 105.99) (width 0.25) (layer F.Cu) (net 1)))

